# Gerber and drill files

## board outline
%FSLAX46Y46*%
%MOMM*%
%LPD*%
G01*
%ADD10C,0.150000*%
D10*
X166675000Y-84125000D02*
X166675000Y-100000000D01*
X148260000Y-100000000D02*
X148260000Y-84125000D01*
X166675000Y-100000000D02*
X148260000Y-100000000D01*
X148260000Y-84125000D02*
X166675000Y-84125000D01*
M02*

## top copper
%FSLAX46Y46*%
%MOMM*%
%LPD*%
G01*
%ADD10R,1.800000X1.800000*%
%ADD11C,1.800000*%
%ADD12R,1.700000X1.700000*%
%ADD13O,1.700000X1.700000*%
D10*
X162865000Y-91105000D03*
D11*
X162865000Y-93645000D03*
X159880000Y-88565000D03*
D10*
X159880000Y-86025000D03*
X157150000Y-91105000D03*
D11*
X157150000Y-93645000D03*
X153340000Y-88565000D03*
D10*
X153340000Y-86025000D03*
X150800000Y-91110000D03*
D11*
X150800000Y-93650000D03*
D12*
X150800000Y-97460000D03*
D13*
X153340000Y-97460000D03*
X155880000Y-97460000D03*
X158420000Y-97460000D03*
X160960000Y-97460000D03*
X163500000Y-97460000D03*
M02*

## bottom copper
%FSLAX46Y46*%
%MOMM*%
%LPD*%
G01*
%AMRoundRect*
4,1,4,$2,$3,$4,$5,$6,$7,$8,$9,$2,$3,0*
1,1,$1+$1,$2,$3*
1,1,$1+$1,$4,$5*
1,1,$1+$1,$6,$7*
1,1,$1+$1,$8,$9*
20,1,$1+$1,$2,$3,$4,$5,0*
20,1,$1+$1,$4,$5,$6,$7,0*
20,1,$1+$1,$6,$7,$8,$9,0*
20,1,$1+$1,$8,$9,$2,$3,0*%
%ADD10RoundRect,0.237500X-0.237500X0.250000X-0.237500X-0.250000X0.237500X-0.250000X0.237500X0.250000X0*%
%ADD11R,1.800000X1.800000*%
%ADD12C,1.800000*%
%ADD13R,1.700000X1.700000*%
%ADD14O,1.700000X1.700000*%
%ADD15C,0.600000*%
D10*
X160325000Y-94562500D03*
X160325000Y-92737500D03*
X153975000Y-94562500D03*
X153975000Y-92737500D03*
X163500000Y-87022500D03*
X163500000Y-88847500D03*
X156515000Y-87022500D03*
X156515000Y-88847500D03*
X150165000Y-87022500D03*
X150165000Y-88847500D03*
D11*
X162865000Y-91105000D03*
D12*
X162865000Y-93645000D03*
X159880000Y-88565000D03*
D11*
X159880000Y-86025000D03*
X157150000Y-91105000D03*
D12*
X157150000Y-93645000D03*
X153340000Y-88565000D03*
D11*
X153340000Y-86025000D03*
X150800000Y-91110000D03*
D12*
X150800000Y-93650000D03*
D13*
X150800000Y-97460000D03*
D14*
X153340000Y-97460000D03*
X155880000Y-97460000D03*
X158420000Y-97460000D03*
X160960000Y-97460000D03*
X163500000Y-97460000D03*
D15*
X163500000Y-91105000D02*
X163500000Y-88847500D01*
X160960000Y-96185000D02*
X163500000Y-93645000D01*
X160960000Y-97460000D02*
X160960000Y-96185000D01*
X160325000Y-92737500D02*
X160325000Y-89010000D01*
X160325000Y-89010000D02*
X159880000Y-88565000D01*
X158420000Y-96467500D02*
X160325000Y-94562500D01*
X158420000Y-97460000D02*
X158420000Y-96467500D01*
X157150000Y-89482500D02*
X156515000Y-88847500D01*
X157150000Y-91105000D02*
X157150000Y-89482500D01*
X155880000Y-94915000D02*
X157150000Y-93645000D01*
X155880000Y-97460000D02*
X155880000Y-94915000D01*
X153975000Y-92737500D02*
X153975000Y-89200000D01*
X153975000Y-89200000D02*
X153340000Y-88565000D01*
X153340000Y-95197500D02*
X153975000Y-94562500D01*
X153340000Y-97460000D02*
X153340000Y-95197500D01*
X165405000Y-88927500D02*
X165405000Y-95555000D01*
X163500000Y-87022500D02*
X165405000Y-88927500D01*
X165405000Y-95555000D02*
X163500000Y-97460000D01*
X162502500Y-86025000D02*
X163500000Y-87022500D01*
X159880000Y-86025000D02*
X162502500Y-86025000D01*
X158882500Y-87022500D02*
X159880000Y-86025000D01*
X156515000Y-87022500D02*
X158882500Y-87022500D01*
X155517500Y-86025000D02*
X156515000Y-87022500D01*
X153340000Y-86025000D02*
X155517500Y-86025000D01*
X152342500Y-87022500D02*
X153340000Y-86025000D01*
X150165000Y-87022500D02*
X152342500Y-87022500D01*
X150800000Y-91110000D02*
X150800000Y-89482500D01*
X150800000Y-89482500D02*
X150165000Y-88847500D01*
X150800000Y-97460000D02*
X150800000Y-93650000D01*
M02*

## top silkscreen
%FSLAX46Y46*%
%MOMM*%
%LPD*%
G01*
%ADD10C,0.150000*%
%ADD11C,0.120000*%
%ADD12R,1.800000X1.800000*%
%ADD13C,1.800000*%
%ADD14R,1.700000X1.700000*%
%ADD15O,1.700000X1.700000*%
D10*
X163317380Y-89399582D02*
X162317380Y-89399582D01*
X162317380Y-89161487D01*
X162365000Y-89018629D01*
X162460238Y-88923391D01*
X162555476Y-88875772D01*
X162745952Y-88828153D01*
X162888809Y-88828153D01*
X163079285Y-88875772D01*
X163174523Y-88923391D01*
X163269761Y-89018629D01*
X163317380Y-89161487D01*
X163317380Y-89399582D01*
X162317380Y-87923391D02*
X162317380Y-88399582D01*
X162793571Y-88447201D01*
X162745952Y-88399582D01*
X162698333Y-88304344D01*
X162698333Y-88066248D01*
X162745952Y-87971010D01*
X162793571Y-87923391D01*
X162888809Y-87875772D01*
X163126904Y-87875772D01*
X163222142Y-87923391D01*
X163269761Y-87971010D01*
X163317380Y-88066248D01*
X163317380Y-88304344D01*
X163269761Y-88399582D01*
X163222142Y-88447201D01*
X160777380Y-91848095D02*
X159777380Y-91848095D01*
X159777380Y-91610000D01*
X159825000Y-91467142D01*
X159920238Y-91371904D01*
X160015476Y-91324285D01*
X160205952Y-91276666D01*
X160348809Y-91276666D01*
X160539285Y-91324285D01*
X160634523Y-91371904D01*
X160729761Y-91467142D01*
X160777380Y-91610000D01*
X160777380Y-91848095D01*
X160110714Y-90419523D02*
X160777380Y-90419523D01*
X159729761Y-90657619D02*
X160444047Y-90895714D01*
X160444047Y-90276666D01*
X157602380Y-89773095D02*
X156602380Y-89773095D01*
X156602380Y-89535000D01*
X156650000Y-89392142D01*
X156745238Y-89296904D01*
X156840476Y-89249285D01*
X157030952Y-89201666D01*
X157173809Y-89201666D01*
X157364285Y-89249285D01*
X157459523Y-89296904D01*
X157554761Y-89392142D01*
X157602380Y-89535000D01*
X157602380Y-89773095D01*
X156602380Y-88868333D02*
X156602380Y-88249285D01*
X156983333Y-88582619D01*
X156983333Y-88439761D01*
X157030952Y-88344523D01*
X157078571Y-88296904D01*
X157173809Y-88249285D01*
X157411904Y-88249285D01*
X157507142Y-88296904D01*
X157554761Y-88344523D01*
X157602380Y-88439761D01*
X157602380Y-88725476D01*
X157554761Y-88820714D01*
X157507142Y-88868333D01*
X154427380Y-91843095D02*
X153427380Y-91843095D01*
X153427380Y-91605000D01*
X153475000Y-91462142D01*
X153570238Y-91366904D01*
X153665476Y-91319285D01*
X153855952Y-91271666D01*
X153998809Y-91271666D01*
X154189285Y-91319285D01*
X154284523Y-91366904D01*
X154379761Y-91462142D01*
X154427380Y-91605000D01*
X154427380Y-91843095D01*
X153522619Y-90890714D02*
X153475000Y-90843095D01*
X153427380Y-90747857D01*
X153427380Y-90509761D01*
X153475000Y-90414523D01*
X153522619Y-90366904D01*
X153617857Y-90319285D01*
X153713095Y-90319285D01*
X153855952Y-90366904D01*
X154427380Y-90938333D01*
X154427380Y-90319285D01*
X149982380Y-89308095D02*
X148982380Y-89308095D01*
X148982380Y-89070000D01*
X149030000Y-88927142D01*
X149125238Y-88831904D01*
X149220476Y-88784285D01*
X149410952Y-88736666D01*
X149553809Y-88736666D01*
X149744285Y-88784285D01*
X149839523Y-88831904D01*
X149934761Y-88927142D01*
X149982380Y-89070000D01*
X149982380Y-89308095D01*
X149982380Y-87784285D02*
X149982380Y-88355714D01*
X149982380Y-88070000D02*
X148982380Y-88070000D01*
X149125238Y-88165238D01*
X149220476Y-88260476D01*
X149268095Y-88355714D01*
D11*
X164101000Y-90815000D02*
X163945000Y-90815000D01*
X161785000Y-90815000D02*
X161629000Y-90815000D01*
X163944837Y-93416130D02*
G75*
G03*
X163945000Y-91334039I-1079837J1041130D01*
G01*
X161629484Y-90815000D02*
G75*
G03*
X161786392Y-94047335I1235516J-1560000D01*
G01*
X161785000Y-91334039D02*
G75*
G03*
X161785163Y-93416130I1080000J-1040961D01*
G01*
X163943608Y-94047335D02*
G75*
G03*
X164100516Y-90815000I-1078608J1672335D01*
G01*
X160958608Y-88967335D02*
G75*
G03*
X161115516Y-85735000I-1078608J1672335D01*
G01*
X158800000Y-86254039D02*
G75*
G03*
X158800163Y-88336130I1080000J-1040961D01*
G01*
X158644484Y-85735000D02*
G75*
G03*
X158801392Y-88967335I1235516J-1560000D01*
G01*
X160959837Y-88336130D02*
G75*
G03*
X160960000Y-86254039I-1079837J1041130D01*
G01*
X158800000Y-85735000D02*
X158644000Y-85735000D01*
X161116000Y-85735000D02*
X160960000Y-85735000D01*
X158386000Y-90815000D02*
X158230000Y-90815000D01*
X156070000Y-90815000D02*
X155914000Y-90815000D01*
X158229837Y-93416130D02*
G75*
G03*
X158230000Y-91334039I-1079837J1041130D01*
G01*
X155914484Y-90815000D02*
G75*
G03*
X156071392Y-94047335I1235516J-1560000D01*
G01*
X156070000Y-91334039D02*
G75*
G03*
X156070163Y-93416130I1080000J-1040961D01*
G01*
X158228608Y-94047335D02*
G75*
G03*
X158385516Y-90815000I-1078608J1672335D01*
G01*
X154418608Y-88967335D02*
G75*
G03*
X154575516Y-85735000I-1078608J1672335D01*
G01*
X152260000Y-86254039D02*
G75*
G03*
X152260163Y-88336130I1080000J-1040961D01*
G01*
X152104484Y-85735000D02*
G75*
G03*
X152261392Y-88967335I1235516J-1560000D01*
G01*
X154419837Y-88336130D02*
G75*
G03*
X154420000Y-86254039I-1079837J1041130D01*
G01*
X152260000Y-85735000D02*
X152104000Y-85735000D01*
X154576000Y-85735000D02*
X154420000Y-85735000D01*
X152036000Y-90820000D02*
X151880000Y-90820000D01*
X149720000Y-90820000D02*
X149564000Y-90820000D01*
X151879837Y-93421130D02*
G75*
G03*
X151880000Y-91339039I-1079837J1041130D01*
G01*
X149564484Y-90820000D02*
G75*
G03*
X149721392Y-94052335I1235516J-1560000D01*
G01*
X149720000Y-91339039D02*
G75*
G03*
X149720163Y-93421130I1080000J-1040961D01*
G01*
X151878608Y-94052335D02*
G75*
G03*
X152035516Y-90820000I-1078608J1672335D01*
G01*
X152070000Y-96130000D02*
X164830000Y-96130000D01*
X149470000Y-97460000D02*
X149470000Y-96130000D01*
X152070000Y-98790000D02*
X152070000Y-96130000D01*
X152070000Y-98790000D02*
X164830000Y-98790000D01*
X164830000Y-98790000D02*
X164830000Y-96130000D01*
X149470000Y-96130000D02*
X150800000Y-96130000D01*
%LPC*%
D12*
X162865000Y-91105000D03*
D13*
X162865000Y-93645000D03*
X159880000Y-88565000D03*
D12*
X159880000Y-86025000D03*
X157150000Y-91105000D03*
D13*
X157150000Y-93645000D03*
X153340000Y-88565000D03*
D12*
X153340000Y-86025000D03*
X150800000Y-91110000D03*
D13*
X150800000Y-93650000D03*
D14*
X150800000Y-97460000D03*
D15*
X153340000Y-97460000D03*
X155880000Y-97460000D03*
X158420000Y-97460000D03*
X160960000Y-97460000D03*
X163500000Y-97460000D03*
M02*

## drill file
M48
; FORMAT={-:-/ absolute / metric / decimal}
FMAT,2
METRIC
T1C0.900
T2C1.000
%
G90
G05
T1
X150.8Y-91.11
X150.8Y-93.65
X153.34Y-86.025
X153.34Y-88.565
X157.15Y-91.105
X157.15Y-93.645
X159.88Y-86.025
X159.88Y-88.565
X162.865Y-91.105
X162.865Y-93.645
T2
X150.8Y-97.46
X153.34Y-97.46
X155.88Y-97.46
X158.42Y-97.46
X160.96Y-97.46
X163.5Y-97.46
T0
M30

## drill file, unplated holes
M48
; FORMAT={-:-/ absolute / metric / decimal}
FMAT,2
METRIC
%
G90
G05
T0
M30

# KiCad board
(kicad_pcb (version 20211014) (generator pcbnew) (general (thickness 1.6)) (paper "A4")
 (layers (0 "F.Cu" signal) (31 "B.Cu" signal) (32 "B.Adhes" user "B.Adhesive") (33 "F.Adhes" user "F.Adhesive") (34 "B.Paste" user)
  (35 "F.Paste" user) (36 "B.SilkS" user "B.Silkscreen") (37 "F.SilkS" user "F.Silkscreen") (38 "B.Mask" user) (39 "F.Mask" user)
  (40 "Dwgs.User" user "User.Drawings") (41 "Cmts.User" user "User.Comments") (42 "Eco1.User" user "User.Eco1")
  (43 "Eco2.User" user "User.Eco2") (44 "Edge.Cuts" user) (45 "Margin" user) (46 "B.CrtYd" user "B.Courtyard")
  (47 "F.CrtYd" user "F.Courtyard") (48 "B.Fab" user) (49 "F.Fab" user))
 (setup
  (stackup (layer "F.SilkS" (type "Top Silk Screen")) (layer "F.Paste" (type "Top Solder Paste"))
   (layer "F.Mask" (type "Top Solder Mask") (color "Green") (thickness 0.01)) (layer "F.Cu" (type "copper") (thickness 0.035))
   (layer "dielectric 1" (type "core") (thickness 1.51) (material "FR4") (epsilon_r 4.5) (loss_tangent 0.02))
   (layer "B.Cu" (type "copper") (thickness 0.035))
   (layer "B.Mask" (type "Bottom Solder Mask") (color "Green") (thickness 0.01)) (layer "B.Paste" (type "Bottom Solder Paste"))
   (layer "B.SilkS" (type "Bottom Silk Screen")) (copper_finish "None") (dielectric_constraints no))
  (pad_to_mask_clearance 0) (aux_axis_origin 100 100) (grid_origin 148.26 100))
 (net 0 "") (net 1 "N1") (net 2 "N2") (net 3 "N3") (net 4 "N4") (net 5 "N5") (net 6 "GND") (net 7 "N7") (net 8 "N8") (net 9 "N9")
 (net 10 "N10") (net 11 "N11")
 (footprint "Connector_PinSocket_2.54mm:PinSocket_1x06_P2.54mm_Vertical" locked (layer "F.Cu") (at 150.8 97.46 90)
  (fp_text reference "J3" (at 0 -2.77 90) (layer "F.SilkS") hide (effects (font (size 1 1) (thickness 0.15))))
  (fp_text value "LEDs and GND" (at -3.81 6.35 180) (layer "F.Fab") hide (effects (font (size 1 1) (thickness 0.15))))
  (fp_line (start 1.33 1.27) (end 1.33 14.03) (layer "F.SilkS") (width 0.12))
  (fp_line (start 0 -1.33) (end 1.33 -1.33) (layer "F.SilkS") (width 0.12))
  (fp_line (start -1.33 1.27) (end 1.33 1.27) (layer "F.SilkS") (width 0.12))
  (fp_line (start -1.33 1.27) (end -1.33 14.03) (layer "F.SilkS") (width 0.12))
  (fp_line (start -1.33 14.03) (end 1.33 14.03) (layer "F.SilkS") (width 0.12))
  (fp_line (start 1.33 -1.33) (end 1.33 0) (layer "F.SilkS") (width 0.12))
  (pad "1" thru_hole rect locked (at 0 0 90) (size 1.7 1.7) (drill 1) (layers *.Cu *.Mask) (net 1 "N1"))
  (pad "2" thru_hole oval locked (at 0 2.54 90) (size 1.7 1.7) (drill 1) (layers *.Cu *.Mask) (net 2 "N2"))
  (pad "3" thru_hole oval locked (at 0 5.08 90) (size 1.7 1.7) (drill 1) (layers *.Cu *.Mask) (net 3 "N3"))
  (pad "4" thru_hole oval locked (at 0 7.62 90) (size 1.7 1.7) (drill 1) (layers *.Cu *.Mask) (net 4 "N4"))
  (pad "5" thru_hole oval locked (at 0 10.16 90) (size 1.7 1.7) (drill 1) (layers *.Cu *.Mask) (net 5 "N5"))
  (pad "6" thru_hole oval locked (at 0 12.7 90) (size 1.7 1.7) (drill 1) (layers *.Cu *.Mask) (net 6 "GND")))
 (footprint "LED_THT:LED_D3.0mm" (layer "F.Cu") (at 157.15 91.105 -90)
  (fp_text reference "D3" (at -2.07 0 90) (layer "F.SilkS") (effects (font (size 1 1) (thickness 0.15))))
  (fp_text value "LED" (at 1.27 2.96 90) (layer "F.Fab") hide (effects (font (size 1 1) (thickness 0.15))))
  (fp_line (start -0.29 1.08) (end -0.29 1.236) (layer "F.SilkS") (width 0.12))
  (fp_line (start -0.29 -1.236) (end -0.29 -1.08) (layer "F.SilkS") (width 0.12))
  (fp_arc (start -0.29 -1.235516) (mid 1.366487 -1.987659) (end 2.942335 -1.078608) (layer "F.SilkS") (width 0.12))
  (fp_arc (start 0.229039 -1.08) (mid 1.270117 -1.5) (end 2.31113 -1.079837) (layer "F.SilkS") (width 0.12))
  (fp_arc (start 2.31113 1.079837) (mid 1.270117 1.5) (end 0.229039 1.08) (layer "F.SilkS") (width 0.12))
  (fp_arc (start 2.942335 1.078608) (mid 1.366487 1.987659) (end -0.29 1.235516) (layer "F.SilkS") (width 0.12))
  (pad "1" thru_hole rect (at 0 0 270) (size 1.8 1.8) (drill 0.9) (layers *.Cu *.Mask) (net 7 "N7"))
  (pad "2" thru_hole circle (at 2.54 0 270) (size 1.8 1.8) (drill 0.9) (layers *.Cu *.Mask) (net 3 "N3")))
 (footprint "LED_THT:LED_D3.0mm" (layer "F.Cu") (at 159.88 86.025 -90)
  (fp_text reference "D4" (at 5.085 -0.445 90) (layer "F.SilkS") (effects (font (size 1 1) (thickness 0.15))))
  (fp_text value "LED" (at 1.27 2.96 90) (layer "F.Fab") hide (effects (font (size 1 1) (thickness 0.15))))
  (fp_line (start -0.29 -1.236) (end -0.29 -1.08) (layer "F.SilkS") (width 0.12))
  (fp_line (start -0.29 1.08) (end -0.29 1.236) (layer "F.SilkS") (width 0.12))
  (fp_arc (start -0.29 -1.235516) (mid 1.366487 -1.987659) (end 2.942335 -1.078608) (layer "F.SilkS") (width 0.12))
  (fp_arc (start 2.942335 1.078608) (mid 1.366487 1.987659) (end -0.29 1.235516) (layer "F.SilkS") (width 0.12))
  (fp_arc (start 0.229039 -1.08) (mid 1.270117 -1.5) (end 2.31113 -1.079837) (layer "F.SilkS") (width 0.12))
  (fp_arc (start 2.31113 1.079837) (mid 1.270117 1.5) (end 0.229039 1.08) (layer "F.SilkS") (width 0.12))
  (pad "1" thru_hole rect (at 0 0 270) (size 1.8 1.8) (drill 0.9) (layers *.Cu *.Mask) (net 6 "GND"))
  (pad "2" thru_hole circle (at 2.54 0 270) (size 1.8 1.8) (drill 0.9) (layers *.Cu *.Mask) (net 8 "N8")))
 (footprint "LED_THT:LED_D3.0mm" (layer "F.Cu") (at 153.34 86.025 -90)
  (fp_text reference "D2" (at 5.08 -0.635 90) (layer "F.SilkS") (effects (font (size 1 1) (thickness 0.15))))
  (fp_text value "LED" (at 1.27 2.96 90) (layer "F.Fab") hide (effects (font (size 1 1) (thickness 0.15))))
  (fp_line (start -0.29 -1.236) (end -0.29 -1.08) (layer "F.SilkS") (width 0.12))
  (fp_line (start -0.29 1.08) (end -0.29 1.236) (layer "F.SilkS") (width 0.12))
  (fp_arc (start 0.229039 -1.08) (mid 1.270117 -1.5) (end 2.31113 -1.079837) (layer "F.SilkS") (width 0.12))
  (fp_arc (start 2.31113 1.079837) (mid 1.270117 1.5) (end 0.229039 1.08) (layer "F.SilkS") (width 0.12))
  (fp_arc (start 2.942335 1.078608) (mid 1.366487 1.987659) (end -0.29 1.235516) (layer "F.SilkS") (width 0.12))
  (fp_arc (start -0.29 -1.235516) (mid 1.366487 -1.987659) (end 2.942335 -1.078608) (layer "F.SilkS") (width 0.12))
  (pad "1" thru_hole rect (at 0 0 270) (size 1.8 1.8) (drill 0.9) (layers *.Cu *.Mask) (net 6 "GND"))
  (pad "2" thru_hole circle (at 2.54 0 270) (size 1.8 1.8) (drill 0.9) (layers *.Cu *.Mask) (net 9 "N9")))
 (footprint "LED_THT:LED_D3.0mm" (layer "F.Cu") (at 150.8 91.11 -90)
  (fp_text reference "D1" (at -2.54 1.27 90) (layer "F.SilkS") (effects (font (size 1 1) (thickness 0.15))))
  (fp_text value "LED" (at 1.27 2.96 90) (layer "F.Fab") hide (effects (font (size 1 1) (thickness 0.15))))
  (fp_line (start -0.29 -1.236) (end -0.29 -1.08) (layer "F.SilkS") (width 0.12))
  (fp_line (start -0.29 1.08) (end -0.29 1.236) (layer "F.SilkS") (width 0.12))
  (fp_arc (start 2.31113 1.079837) (mid 1.270117 1.5) (end 0.229039 1.08) (layer "F.SilkS") (width 0.12))
  (fp_arc (start -0.29 -1.235516) (mid 1.366487 -1.987659) (end 2.942335 -1.078608) (layer "F.SilkS") (width 0.12))
  (fp_arc (start 2.942335 1.078608) (mid 1.366487 1.987659) (end -0.29 1.235516) (layer "F.SilkS") (width 0.12))
  (fp_arc (start 0.229039 -1.08) (mid 1.270117 -1.5) (end 2.31113 -1.079837) (layer "F.SilkS") (width 0.12))
  (pad "1" thru_hole rect (at 0 0 270) (size 1.8 1.8) (drill 0.9) (layers *.Cu *.Mask) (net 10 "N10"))
  (pad "2" thru_hole circle (at 2.54 0 270) (size 1.8 1.8) (drill 0.9) (layers *.Cu *.Mask) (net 1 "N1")))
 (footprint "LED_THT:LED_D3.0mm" (layer "F.Cu") (at 162.865 91.105 -90)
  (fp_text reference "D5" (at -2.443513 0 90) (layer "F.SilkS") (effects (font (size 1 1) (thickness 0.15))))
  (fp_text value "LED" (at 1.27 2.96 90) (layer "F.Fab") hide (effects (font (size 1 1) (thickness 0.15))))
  (fp_line (start -0.29 -1.236) (end -0.29 -1.08) (layer "F.SilkS") (width 0.12))
  (fp_line (start -0.29 1.08) (end -0.29 1.236) (layer "F.SilkS") (width 0.12))
  (fp_arc (start 2.942335 1.078608) (mid 1.366487 1.987659) (end -0.29 1.235516) (layer "F.SilkS") (width 0.12))
  (fp_arc (start -0.29 -1.235516) (mid 1.366487 -1.987659) (end 2.942335 -1.078608) (layer "F.SilkS") (width 0.12))
  (fp_arc (start 0.229039 -1.08) (mid 1.270117 -1.5) (end 2.31113 -1.079837) (layer "F.SilkS") (width 0.12))
  (fp_arc (start 2.31113 1.079837) (mid 1.270117 1.5) (end 0.229039 1.08) (layer "F.SilkS") (width 0.12))
  (pad "1" thru_hole rect (at 0 0 270) (size 1.8 1.8) (drill 0.9) (layers *.Cu *.Mask) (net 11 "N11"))
  (pad "2" thru_hole circle (at 2.54 0 270) (size 1.8 1.8) (drill 0.9) (layers *.Cu *.Mask) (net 5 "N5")))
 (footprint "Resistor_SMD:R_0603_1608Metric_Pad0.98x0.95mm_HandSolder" (layer "B.Cu") (at 160.325 93.65 -90)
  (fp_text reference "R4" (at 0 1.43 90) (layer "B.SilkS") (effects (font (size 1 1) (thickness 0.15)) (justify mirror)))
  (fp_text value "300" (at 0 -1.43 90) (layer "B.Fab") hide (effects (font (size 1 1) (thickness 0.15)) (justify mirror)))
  (pad "1" smd roundrect (at -0.9125 0 270) (size 0.975 0.95) (layers "B.Cu" "B.Paste" "B.Mask") (roundrect_rratio 0.25) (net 8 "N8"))
  (pad "2" smd roundrect (at 0.9125 0 270) (size 0.975 0.95) (layers "B.Cu" "B.Paste" "B.Mask") (roundrect_rratio 0.25) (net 4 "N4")))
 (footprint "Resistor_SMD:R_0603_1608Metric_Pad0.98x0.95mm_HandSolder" (layer "B.Cu") (at 163.5 87.935 -90)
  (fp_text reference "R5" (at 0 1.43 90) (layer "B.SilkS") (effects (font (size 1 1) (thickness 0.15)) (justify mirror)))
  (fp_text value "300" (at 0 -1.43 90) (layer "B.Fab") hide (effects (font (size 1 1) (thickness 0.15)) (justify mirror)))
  (pad "1" smd roundrect (at -0.9125 0 270) (size 0.975 0.95) (layers "B.Cu" "B.Paste" "B.Mask") (roundrect_rratio 0.25) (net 6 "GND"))
  (pad "2" smd roundrect (at 0.9125 0 270) (size 0.975 0.95) (layers "B.Cu" "B.Paste" "B.Mask") (roundrect_rratio 0.25) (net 11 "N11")))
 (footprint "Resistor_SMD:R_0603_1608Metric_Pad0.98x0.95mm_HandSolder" (layer "B.Cu") (at 153.975 93.65 -90)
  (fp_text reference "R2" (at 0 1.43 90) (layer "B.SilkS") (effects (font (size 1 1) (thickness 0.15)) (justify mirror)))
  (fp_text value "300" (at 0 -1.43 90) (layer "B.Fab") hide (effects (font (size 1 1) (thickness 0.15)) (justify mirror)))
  (pad "1" smd roundrect (at -0.9125 0 270) (size 0.975 0.95) (layers "B.Cu" "B.Paste" "B.Mask") (roundrect_rratio 0.25) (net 9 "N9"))
  (pad "2" smd roundrect (at 0.9125 0 270) (size 0.975 0.95) (layers "B.Cu" "B.Paste" "B.Mask") (roundrect_rratio 0.25) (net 2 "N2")))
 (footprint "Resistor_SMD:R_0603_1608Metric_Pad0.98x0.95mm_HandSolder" (layer "B.Cu") (at 156.515 87.935 -90)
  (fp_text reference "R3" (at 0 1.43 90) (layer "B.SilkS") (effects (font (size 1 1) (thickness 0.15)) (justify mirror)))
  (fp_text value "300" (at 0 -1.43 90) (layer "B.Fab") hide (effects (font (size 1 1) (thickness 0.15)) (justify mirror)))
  (pad "1" smd roundrect (at -0.9125 0 270) (size 0.975 0.95) (layers "B.Cu" "B.Paste" "B.Mask") (roundrect_rratio 0.25) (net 6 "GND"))
  (pad "2" smd roundrect (at 0.9125 0 270) (size 0.975 0.95) (layers "B.Cu" "B.Paste" "B.Mask") (roundrect_rratio 0.25) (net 7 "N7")))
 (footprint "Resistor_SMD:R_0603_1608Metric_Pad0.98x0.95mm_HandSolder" (layer "B.Cu") (at 150.165 87.935 -90)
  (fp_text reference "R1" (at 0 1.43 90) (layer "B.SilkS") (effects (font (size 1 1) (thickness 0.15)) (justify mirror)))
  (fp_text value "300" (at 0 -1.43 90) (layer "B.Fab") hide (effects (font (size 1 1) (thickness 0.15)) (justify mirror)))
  (pad "1" smd roundrect (at -0.9125 0 270) (size 0.975 0.95) (layers "B.Cu" "B.Paste" "B.Mask") (roundrect_rratio 0.25) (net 6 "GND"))
  (pad "2" smd roundrect (at 0.9125 0 270) (size 0.975 0.95) (layers "B.Cu" "B.Paste" "B.Mask") (roundrect_rratio 0.25) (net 10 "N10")))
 (gr_line (start 148.26 100) (end 148.26 84.125) (layer "Edge.Cuts") (width 0.15))
 (gr_line (start 166.675 84.125) (end 166.675 100) (layer "Edge.Cuts") (width 0.15))
 (gr_line (start 166.675 100) (end 148.26 100) (layer "Edge.Cuts") (width 0.15))
 (gr_line (start 148.26 84.125) (end 166.675 84.125) (layer "Edge.Cuts") (width 0.15))
 (segment (start 150.8 89.4825) (end 150.165 88.8475) (width 0.6) (layer "B.Cu") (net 10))
 (segment (start 150.8 91.11) (end 150.8 89.4825) (width 0.6) (layer "B.Cu") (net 10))
 (segment (start 150.8 97.46) (end 150.8 93.65) (width 0.6) (layer "B.Cu") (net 1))
 (segment (start 153.34 97.46) (end 153.34 95.1975) (width 0.6) (layer "B.Cu") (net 2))
 (segment (start 153.34 95.1975) (end 153.975 94.5625) (width 0.6) (layer "B.Cu") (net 2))
 (segment (start 157.15 89.4825) (end 156.515 88.8475) (width 0.6) (layer "B.Cu") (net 7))
 (segment (start 157.15 91.105) (end 157.15 89.4825) (width 0.6) (layer "B.Cu") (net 7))
 (segment (start 155.88 97.46) (end 155.88 94.915) (width 0.6) (layer "B.Cu") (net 3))
 (segment (start 155.88 94.915) (end 157.15 93.645) (width 0.6) (layer "B.Cu") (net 3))
 (segment (start 158.42 97.46) (end 158.42 96.4675) (width 0.6) (layer "B.Cu") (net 4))
 (segment (start 158.42 96.4675) (end 160.325 94.5625) (width 0.6) (layer "B.Cu") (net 4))
 (segment (start 163.5 91.105) (end 163.5 88.8475) (width 0.6) (layer "B.Cu") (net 11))
 (segment (start 160.96 97.46) (end 160.96 96.185) (width 0.6) (layer "B.Cu") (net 5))
 (segment (start 160.96 96.185) (end 163.5 93.645) (width 0.6) (layer "B.Cu") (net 5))
 (segment (start 158.8825 87.0225) (end 159.88 86.025) (width 0.6) (layer "B.Cu") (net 6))
 (segment (start 152.3425 87.0225) (end 153.34 86.025) (width 0.6) (layer "B.Cu") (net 6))
 (segment (start 153.34 86.025) (end 155.5175 86.025) (width 0.6) (layer "B.Cu") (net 6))
 (segment (start 165.405 88.9275) (end 165.405 95.555) (width 0.6) (layer "B.Cu") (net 6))
 (segment (start 163.5 87.0225) (end 165.405 88.9275) (width 0.6) (layer "B.Cu") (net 6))
 (segment (start 150.165 87.0225) (end 152.3425 87.0225) (width 0.6) (layer "B.Cu") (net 6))
 (segment (start 159.88 86.025) (end 162.5025 86.025) (width 0.6) (layer "B.Cu") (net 6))
 (segment (start 155.5175 86.025) (end 156.515 87.0225) (width 0.6) (layer "B.Cu") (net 6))
 (segment (start 165.405 95.555) (end 163.5 97.46) (width 0.6) (layer "B.Cu") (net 6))
 (segment (start 156.515 87.0225) (end 158.8825 87.0225) (width 0.6) (layer "B.Cu") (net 6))
 (segment (start 162.5025 86.025) (end 163.5 87.0225) (width 0.6) (layer "B.Cu") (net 6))
 (segment (start 153.975 89.2) (end 153.34 88.565) (width 0.6) (layer "B.Cu") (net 9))
 (segment (start 153.975 92.7375) (end 153.975 89.2) (width 0.6) (layer "B.Cu") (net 9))
 (segment (start 160.325 92.7375) (end 160.325 89.01) (width 0.6) (layer "B.Cu") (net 8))
 (segment (start 160.325 89.01) (end 159.88 88.565) (width 0.6) (layer "B.Cu") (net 8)))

